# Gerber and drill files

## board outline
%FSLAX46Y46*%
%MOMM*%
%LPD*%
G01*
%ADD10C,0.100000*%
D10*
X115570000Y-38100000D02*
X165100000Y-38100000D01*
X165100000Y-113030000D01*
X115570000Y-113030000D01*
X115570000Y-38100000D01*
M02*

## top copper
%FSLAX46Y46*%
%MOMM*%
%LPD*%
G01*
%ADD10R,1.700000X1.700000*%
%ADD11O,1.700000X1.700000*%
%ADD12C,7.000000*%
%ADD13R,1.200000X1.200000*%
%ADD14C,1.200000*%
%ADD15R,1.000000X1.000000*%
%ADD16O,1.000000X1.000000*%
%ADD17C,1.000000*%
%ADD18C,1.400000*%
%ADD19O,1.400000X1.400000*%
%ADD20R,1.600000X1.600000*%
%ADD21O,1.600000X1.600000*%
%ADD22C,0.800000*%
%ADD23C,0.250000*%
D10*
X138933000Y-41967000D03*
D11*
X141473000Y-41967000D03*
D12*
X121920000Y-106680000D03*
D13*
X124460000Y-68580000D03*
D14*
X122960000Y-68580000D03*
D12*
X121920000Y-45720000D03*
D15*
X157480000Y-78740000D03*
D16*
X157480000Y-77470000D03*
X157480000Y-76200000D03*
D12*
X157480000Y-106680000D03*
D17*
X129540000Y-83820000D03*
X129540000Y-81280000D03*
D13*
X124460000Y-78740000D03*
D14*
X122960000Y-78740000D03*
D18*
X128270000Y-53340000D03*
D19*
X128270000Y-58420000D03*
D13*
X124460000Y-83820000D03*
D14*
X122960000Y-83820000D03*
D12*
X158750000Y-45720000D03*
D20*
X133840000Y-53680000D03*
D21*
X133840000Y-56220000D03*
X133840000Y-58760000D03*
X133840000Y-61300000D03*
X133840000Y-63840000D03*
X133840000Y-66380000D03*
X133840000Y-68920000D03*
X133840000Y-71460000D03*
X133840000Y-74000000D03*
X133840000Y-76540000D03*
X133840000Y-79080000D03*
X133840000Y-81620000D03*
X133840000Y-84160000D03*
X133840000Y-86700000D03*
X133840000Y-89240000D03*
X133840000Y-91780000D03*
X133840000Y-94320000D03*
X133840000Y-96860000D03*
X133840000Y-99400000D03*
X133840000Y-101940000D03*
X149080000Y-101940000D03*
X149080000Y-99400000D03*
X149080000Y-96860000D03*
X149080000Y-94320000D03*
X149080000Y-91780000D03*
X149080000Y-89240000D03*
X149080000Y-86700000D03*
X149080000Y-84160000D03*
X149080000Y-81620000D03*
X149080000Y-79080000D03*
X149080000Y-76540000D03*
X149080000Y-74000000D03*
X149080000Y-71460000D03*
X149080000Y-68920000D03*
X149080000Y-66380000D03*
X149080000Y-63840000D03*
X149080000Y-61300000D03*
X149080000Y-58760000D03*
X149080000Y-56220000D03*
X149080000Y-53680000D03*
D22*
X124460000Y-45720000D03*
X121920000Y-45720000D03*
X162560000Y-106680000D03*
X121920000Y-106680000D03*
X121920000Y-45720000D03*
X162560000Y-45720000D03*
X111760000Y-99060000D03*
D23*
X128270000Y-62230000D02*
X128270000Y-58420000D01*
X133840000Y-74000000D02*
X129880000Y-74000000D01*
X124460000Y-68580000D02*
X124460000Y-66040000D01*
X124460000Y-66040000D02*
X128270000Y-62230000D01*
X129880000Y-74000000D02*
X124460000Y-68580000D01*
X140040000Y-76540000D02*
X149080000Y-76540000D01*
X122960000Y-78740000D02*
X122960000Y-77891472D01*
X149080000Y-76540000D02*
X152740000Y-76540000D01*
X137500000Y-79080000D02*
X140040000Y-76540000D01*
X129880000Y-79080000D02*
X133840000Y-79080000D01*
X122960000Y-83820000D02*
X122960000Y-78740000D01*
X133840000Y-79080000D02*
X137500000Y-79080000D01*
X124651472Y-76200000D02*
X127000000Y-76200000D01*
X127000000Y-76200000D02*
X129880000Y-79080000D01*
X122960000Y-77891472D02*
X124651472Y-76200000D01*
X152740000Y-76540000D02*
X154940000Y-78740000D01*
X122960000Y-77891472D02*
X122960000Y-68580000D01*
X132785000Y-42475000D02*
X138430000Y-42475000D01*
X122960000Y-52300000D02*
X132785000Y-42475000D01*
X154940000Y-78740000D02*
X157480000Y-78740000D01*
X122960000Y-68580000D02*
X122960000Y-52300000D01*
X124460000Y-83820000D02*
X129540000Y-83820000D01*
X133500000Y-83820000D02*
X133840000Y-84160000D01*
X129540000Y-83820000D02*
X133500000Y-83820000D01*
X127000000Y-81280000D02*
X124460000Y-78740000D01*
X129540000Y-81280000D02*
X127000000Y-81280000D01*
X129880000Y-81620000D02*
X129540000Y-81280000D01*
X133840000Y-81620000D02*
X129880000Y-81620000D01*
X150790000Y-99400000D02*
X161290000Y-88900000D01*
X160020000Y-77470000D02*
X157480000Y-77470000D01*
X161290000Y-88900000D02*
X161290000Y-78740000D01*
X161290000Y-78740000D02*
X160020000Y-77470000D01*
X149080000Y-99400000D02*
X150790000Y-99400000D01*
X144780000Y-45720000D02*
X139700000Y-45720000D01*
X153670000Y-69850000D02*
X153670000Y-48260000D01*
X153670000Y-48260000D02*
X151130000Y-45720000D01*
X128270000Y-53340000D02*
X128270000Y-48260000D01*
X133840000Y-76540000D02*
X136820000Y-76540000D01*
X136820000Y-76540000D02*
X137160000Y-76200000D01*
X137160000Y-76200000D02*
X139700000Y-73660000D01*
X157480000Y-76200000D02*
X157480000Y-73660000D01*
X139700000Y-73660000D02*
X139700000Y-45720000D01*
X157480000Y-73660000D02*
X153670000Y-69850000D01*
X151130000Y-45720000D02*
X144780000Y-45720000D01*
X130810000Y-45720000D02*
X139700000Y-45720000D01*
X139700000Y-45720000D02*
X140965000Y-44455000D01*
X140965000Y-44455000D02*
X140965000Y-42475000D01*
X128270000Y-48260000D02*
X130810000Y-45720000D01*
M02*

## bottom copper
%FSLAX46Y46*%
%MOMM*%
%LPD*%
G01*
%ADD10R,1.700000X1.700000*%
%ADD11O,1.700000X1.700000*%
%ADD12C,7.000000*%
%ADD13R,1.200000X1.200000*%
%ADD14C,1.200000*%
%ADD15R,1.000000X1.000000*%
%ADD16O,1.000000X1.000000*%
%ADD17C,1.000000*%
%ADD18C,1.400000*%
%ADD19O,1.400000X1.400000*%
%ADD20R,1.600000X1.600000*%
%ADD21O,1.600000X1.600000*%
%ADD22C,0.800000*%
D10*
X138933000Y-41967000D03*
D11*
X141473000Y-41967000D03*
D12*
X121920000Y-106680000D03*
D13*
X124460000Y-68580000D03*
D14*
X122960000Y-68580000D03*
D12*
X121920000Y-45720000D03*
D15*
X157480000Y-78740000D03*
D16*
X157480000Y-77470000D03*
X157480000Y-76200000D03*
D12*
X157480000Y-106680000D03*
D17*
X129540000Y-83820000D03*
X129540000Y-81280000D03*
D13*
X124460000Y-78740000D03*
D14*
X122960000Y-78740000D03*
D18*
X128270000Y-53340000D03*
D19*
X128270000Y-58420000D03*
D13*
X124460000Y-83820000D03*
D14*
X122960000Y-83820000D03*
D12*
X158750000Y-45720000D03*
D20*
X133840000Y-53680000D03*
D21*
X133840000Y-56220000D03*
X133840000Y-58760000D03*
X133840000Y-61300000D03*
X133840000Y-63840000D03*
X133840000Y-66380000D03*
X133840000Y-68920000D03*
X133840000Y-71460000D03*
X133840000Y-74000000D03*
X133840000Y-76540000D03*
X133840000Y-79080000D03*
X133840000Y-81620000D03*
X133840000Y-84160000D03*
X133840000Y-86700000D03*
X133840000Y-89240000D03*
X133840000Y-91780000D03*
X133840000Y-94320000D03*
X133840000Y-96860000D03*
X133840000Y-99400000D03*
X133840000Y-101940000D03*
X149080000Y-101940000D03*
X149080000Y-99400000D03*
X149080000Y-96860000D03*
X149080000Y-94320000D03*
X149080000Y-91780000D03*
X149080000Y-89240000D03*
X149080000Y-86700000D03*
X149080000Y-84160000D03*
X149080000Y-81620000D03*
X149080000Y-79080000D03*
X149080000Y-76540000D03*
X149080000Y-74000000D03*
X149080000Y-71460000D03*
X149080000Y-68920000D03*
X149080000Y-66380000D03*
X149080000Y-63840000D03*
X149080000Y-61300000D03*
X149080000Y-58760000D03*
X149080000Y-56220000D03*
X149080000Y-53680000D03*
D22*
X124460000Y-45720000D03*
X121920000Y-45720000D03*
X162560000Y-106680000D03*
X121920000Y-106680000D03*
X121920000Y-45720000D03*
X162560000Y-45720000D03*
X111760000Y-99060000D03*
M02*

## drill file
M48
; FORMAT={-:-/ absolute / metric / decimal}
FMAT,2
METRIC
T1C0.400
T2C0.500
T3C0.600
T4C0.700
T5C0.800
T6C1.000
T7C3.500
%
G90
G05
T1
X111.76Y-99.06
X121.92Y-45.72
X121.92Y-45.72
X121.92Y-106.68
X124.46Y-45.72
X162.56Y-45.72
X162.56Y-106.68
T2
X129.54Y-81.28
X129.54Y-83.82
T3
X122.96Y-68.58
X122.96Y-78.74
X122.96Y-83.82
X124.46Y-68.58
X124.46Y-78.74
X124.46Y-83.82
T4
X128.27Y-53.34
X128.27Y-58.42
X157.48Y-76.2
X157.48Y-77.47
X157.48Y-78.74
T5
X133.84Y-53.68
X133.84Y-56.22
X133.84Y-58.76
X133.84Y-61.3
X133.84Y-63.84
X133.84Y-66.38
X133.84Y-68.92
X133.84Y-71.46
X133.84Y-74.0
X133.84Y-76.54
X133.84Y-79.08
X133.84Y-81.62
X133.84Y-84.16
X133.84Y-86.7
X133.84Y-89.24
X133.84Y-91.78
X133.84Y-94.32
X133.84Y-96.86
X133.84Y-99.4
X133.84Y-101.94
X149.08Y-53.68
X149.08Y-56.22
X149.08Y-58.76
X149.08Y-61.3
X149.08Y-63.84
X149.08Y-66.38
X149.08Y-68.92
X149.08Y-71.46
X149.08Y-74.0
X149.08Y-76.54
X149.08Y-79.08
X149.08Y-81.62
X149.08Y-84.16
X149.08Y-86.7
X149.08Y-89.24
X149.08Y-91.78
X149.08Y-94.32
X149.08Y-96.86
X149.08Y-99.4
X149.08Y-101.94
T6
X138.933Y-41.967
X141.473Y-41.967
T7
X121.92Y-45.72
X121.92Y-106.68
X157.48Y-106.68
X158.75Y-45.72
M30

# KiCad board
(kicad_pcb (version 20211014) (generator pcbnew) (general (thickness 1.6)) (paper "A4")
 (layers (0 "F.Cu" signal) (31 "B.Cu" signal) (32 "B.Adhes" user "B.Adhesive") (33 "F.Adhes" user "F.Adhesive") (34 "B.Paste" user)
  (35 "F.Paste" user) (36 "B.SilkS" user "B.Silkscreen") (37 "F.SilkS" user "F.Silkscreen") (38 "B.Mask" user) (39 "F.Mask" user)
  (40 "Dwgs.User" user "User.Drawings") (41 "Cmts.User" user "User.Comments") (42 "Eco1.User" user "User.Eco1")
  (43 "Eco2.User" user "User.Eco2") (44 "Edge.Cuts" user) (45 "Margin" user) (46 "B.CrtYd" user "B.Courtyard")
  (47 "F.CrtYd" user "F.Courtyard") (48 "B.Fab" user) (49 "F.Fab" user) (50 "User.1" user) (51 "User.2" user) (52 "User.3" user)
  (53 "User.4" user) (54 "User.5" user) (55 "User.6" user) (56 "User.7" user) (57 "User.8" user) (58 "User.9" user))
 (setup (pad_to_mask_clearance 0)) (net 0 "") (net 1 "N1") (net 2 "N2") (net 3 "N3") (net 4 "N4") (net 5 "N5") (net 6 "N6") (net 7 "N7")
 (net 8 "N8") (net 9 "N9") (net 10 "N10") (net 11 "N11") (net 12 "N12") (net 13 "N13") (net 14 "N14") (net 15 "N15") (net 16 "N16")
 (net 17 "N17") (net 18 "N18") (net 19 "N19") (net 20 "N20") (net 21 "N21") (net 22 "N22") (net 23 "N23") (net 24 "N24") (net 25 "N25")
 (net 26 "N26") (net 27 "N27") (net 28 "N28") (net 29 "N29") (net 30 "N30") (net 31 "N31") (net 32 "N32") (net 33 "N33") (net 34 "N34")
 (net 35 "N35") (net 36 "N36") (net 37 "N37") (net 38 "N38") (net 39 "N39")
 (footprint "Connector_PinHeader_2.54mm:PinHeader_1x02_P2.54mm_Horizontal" (layer "F.Cu") (at 138.933 41.967 90)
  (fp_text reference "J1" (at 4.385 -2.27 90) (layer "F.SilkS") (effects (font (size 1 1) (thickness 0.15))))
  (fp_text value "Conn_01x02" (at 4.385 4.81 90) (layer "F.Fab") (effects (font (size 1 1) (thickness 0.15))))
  (pad "1" thru_hole rect (at 0 0 90) (size 1.7 1.7) (drill 1) (layers *.Cu *.Mask) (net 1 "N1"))
  (pad "2" thru_hole oval (at 0 2.54 90) (size 1.7 1.7) (drill 1) (layers *.Cu *.Mask) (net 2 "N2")))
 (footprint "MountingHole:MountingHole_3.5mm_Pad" (layer "F.Cu") (at 121.92 106.68)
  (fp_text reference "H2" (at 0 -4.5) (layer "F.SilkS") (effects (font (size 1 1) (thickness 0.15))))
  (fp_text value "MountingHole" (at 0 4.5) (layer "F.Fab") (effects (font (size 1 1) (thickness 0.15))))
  (pad "1" thru_hole circle (at 0 0) (size 7 7) (drill 3.5) (layers *.Cu *.Mask)))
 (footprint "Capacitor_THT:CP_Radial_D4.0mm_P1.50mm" (layer "F.Cu") (at 124.46 68.58 180)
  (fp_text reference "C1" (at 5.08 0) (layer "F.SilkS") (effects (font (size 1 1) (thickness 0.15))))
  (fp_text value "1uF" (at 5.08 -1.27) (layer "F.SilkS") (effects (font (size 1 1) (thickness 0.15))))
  (pad "1" thru_hole rect (at 0 0 180) (size 1.2 1.2) (drill 0.6) (layers *.Cu *.Mask) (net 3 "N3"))
  (pad "2" thru_hole circle (at 1.5 0 180) (size 1.2 1.2) (drill 0.6) (layers *.Cu *.Mask) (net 1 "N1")))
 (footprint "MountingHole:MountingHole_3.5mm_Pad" (layer "F.Cu") (at 121.92 45.72)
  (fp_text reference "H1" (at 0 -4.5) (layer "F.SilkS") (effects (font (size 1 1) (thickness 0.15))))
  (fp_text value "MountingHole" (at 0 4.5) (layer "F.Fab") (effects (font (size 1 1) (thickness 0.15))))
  (pad "1" thru_hole circle (at 0 0) (size 7 7) (drill 3.5) (layers *.Cu *.Mask)))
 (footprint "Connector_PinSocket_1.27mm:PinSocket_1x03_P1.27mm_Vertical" (layer "F.Cu") (at 157.48 78.74 180)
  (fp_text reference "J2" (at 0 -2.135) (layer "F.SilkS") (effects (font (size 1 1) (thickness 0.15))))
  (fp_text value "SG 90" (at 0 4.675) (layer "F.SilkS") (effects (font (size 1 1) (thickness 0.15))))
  (pad "1" thru_hole rect (at 0 0 180) (size 1 1) (drill 0.7) (layers *.Cu *.Mask) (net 1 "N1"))
  (pad "2" thru_hole oval (at 0 1.27 180) (size 1 1) (drill 0.7) (layers *.Cu *.Mask) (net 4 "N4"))
  (pad "3" thru_hole oval (at 0 2.54 180) (size 1 1) (drill 0.7) (layers *.Cu *.Mask) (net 2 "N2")))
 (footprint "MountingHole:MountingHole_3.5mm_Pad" (layer "F.Cu") (at 157.48 106.68)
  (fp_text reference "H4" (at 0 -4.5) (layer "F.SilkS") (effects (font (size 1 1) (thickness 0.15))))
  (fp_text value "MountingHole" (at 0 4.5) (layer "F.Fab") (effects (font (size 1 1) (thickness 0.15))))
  (pad "1" thru_hole circle (at 0 0) (size 7 7) (drill 3.5) (layers *.Cu *.Mask)))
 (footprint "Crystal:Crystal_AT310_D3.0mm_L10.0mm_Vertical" (layer "F.Cu") (at 129.54 83.82 90)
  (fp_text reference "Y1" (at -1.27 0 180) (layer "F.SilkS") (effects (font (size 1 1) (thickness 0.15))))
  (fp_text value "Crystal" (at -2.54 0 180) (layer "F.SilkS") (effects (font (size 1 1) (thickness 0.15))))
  (pad "1" thru_hole circle (at 0 0 90) (size 1 1) (drill 0.5) (layers *.Cu *.Mask) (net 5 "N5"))
  (pad "2" thru_hole circle (at 2.54 0 90) (size 1 1) (drill 0.5) (layers *.Cu *.Mask) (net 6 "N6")))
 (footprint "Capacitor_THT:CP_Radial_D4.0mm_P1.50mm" (layer "F.Cu") (at 124.46 78.74 180)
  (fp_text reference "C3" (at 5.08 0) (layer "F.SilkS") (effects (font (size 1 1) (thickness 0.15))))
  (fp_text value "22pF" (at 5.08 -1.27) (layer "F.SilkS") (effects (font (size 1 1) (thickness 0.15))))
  (pad "1" thru_hole rect (at 0 0 180) (size 1.2 1.2) (drill 0.6) (layers *.Cu *.Mask) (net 6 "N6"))
  (pad "2" thru_hole circle (at 1.5 0 180) (size 1.2 1.2) (drill 0.6) (layers *.Cu *.Mask) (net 1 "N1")))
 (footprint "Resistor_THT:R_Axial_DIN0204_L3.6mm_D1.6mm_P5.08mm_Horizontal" (layer "F.Cu") (at 128.27 53.34 -90)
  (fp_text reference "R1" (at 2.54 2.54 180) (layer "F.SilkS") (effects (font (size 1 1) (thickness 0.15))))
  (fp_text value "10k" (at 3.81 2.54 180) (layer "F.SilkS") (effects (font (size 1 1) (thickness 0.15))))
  (pad "1" thru_hole circle (at 0 0 270) (size 1.4 1.4) (drill 0.7) (layers *.Cu *.Mask) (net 2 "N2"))
  (pad "2" thru_hole oval (at 5.08 0 270) (size 1.4 1.4) (drill 0.7) (layers *.Cu *.Mask) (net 3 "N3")))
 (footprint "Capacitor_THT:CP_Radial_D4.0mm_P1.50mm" (layer "F.Cu") (at 124.46 83.82 180)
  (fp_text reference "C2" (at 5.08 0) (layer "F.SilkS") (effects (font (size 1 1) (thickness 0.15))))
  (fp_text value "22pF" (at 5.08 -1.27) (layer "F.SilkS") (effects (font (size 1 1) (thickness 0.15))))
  (pad "1" thru_hole rect (at 0 0 180) (size 1.2 1.2) (drill 0.6) (layers *.Cu *.Mask) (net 5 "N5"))
  (pad "2" thru_hole circle (at 1.5 0 180) (size 1.2 1.2) (drill 0.6) (layers *.Cu *.Mask) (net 1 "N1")))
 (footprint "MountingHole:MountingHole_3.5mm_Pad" (layer "F.Cu") (at 158.75 45.72)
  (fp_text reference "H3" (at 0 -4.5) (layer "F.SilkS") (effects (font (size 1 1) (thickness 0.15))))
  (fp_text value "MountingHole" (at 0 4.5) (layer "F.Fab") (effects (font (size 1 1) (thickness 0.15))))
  (pad "1" thru_hole circle (at 0 0) (size 7 7) (drill 3.5) (layers *.Cu *.Mask)))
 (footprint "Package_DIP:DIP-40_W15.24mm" (layer "F.Cu") (at 133.84 53.68)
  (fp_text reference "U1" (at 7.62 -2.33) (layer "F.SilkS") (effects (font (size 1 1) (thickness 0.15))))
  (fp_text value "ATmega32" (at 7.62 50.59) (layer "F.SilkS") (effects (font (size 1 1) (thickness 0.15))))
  (pad "1" thru_hole rect (at 0 0) (size 1.6 1.6) (drill 0.8) (layers *.Cu *.Mask) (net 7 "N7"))
  (pad "2" thru_hole oval (at 0 2.54) (size 1.6 1.6) (drill 0.8) (layers *.Cu *.Mask) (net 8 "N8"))
  (pad "3" thru_hole oval (at 0 5.08) (size 1.6 1.6) (drill 0.8) (layers *.Cu *.Mask) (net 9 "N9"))
  (pad "4" thru_hole oval (at 0 7.62) (size 1.6 1.6) (drill 0.8) (layers *.Cu *.Mask) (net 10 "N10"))
  (pad "5" thru_hole oval (at 0 10.16) (size 1.6 1.6) (drill 0.8) (layers *.Cu *.Mask) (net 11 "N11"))
  (pad "6" thru_hole oval (at 0 12.7) (size 1.6 1.6) (drill 0.8) (layers *.Cu *.Mask) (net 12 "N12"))
  (pad "7" thru_hole oval (at 0 15.24) (size 1.6 1.6) (drill 0.8) (layers *.Cu *.Mask) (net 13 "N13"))
  (pad "8" thru_hole oval (at 0 17.78) (size 1.6 1.6) (drill 0.8) (layers *.Cu *.Mask) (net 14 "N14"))
  (pad "9" thru_hole oval (at 0 20.32) (size 1.6 1.6) (drill 0.8) (layers *.Cu *.Mask) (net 3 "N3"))
  (pad "10" thru_hole oval (at 0 22.86) (size 1.6 1.6) (drill 0.8) (layers *.Cu *.Mask) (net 2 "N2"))
  (pad "11" thru_hole oval (at 0 25.4) (size 1.6 1.6) (drill 0.8) (layers *.Cu *.Mask) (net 1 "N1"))
  (pad "12" thru_hole oval (at 0 27.94) (size 1.6 1.6) (drill 0.8) (layers *.Cu *.Mask) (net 6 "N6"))
  (pad "13" thru_hole oval (at 0 30.48) (size 1.6 1.6) (drill 0.8) (layers *.Cu *.Mask) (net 5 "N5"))
  (pad "14" thru_hole oval (at 0 33.02) (size 1.6 1.6) (drill 0.8) (layers *.Cu *.Mask) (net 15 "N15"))
  (pad "15" thru_hole oval (at 0 35.56) (size 1.6 1.6) (drill 0.8) (layers *.Cu *.Mask) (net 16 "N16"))
  (pad "16" thru_hole oval (at 0 38.1) (size 1.6 1.6) (drill 0.8) (layers *.Cu *.Mask) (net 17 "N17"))
  (pad "17" thru_hole oval (at 0 40.64) (size 1.6 1.6) (drill 0.8) (layers *.Cu *.Mask) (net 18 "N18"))
  (pad "18" thru_hole oval (at 0 43.18) (size 1.6 1.6) (drill 0.8) (layers *.Cu *.Mask) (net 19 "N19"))
  (pad "19" thru_hole oval (at 0 45.72) (size 1.6 1.6) (drill 0.8) (layers *.Cu *.Mask) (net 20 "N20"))
  (pad "20" thru_hole oval (at 0 48.26) (size 1.6 1.6) (drill 0.8) (layers *.Cu *.Mask) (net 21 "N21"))
  (pad "21" thru_hole oval (at 15.24 48.26) (size 1.6 1.6) (drill 0.8) (layers *.Cu *.Mask) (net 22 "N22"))
  (pad "22" thru_hole oval (at 15.24 45.72) (size 1.6 1.6) (drill 0.8) (layers *.Cu *.Mask) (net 4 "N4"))
  (pad "23" thru_hole oval (at 15.24 43.18) (size 1.6 1.6) (drill 0.8) (layers *.Cu *.Mask) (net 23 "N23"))
  (pad "24" thru_hole oval (at 15.24 40.64) (size 1.6 1.6) (drill 0.8) (layers *.Cu *.Mask) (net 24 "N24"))
  (pad "25" thru_hole oval (at 15.24 38.1) (size 1.6 1.6) (drill 0.8) (layers *.Cu *.Mask) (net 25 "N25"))
  (pad "26" thru_hole oval (at 15.24 35.56) (size 1.6 1.6) (drill 0.8) (layers *.Cu *.Mask) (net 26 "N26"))
  (pad "27" thru_hole oval (at 15.24 33.02) (size 1.6 1.6) (drill 0.8) (layers *.Cu *.Mask) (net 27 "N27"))
  (pad "28" thru_hole oval (at 15.24 30.48) (size 1.6 1.6) (drill 0.8) (layers *.Cu *.Mask) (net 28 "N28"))
  (pad "29" thru_hole oval (at 15.24 27.94) (size 1.6 1.6) (drill 0.8) (layers *.Cu *.Mask) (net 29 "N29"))
  (pad "30" thru_hole oval (at 15.24 25.4) (size 1.6 1.6) (drill 0.8) (layers *.Cu *.Mask) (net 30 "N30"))
  (pad "31" thru_hole oval (at 15.24 22.86) (size 1.6 1.6) (drill 0.8) (layers *.Cu *.Mask) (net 1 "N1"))
  (pad "32" thru_hole oval (at 15.24 20.32) (size 1.6 1.6) (drill 0.8) (layers *.Cu *.Mask) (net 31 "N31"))
  (pad "33" thru_hole oval (at 15.24 17.78) (size 1.6 1.6) (drill 0.8) (layers *.Cu *.Mask) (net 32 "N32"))
  (pad "34" thru_hole oval (at 15.24 15.24) (size 1.6 1.6) (drill 0.8) (layers *.Cu *.Mask) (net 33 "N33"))
  (pad "35" thru_hole oval (at 15.24 12.7) (size 1.6 1.6) (drill 0.8) (layers *.Cu *.Mask) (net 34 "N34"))
  (pad "36" thru_hole oval (at 15.24 10.16) (size 1.6 1.6) (drill 0.8) (layers *.Cu *.Mask) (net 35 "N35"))
  (pad "37" thru_hole oval (at 15.24 7.62) (size 1.6 1.6) (drill 0.8) (layers *.Cu *.Mask) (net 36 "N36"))
  (pad "38" thru_hole oval (at 15.24 5.08) (size 1.6 1.6) (drill 0.8) (layers *.Cu *.Mask) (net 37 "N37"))
  (pad "39" thru_hole oval (at 15.24 2.54) (size 1.6 1.6) (drill 0.8) (layers *.Cu *.Mask) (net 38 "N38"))
  (pad "40" thru_hole oval (at 15.24 0) (size 1.6 1.6) (drill 0.8) (layers *.Cu *.Mask) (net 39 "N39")))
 (gr_rect (start 115.57 38.1) (end 165.1 113.03) (layer "Edge.Cuts") (width 0.1) (fill none))
 (via (at 124.46 45.72) (size 0.8) (drill 0.4) (layers "F.Cu" "B.Cu") (free) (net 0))
 (via (at 121.92 45.72) (size 0.8) (drill 0.4) (layers "F.Cu" "B.Cu") (free) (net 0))
 (via (at 162.56 106.68) (size 0.8) (drill 0.4) (layers "F.Cu" "B.Cu") (free) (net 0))
 (via (at 121.92 106.68) (size 0.8) (drill 0.4) (layers "F.Cu" "B.Cu") (free) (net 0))
 (via (at 121.92 45.72) (size 0.8) (drill 0.4) (layers "F.Cu" "B.Cu") (free) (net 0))
 (via (at 162.56 45.72) (size 0.8) (drill 0.4) (layers "F.Cu" "B.Cu") (free) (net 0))
 (via (at 111.76 99.06) (size 0.8) (drill 0.4) (layers "F.Cu" "B.Cu") (free) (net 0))
 (segment (start 128.27 62.23) (end 128.27 58.42) (width 0.25) (layer "F.Cu") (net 3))
 (segment (start 133.84 74) (end 129.88 74) (width 0.25) (layer "F.Cu") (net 3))
 (segment (start 124.46 68.58) (end 124.46 66.04) (width 0.25) (layer "F.Cu") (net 3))
 (segment (start 124.46 66.04) (end 128.27 62.23) (width 0.25) (layer "F.Cu") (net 3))
 (segment (start 129.88 74) (end 124.46 68.58) (width 0.25) (layer "F.Cu") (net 3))
 (segment (start 140.04 76.54) (end 149.08 76.54) (width 0.25) (layer "F.Cu") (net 1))
 (segment (start 122.96 78.74) (end 122.96 77.891472) (width 0.25) (layer "F.Cu") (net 1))
 (segment (start 149.08 76.54) (end 152.74 76.54) (width 0.25) (layer "F.Cu") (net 1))
 (segment (start 137.5 79.08) (end 140.04 76.54) (width 0.25) (layer "F.Cu") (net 1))
 (segment (start 129.88 79.08) (end 133.84 79.08) (width 0.25) (layer "F.Cu") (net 1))
 (segment (start 122.96 83.82) (end 122.96 78.74) (width 0.25) (layer "F.Cu") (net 1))
 (segment (start 133.84 79.08) (end 137.5 79.08) (width 0.25) (layer "F.Cu") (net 1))
 (segment (start 124.651472 76.2) (end 127 76.2) (width 0.25) (layer "F.Cu") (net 1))
 (segment (start 127 76.2) (end 129.88 79.08) (width 0.25) (layer "F.Cu") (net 1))
 (segment (start 122.96 77.891472) (end 124.651472 76.2) (width 0.25) (layer "F.Cu") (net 1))
 (segment (start 152.74 76.54) (end 154.94 78.74) (width 0.25) (layer "F.Cu") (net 1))
 (segment (start 122.96 77.891472) (end 122.96 68.58) (width 0.25) (layer "F.Cu") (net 1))
 (segment (start 132.785 42.475) (end 138.43 42.475) (width 0.25) (layer "F.Cu") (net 1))
 (segment (start 122.96 52.3) (end 132.785 42.475) (width 0.25) (layer "F.Cu") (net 1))
 (segment (start 154.94 78.74) (end 157.48 78.74) (width 0.25) (layer "F.Cu") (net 1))
 (segment (start 122.96 68.58) (end 122.96 52.3) (width 0.25) (layer "F.Cu") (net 1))
 (segment (start 124.46 83.82) (end 129.54 83.82) (width 0.25) (layer "F.Cu") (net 5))
 (segment (start 133.5 83.82) (end 133.84 84.16) (width 0.25) (layer "F.Cu") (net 5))
 (segment (start 129.54 83.82) (end 133.5 83.82) (width 0.25) (layer "F.Cu") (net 5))
 (segment (start 127 81.28) (end 124.46 78.74) (width 0.25) (layer "F.Cu") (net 6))
 (segment (start 129.54 81.28) (end 127 81.28) (width 0.25) (layer "F.Cu") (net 6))
 (segment (start 129.88 81.62) (end 129.54 81.28) (width 0.25) (layer "F.Cu") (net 6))
 (segment (start 133.84 81.62) (end 129.88 81.62) (width 0.25) (layer "F.Cu") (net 6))
 (segment (start 150.79 99.4) (end 161.29 88.9) (width 0.25) (layer "F.Cu") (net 4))
 (segment (start 160.02 77.47) (end 157.48 77.47) (width 0.25) (layer "F.Cu") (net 4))
 (segment (start 161.29 88.9) (end 161.29 78.74) (width 0.25) (layer "F.Cu") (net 4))
 (segment (start 161.29 78.74) (end 160.02 77.47) (width 0.25) (layer "F.Cu") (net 4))
 (segment (start 149.08 99.4) (end 150.79 99.4) (width 0.25) (layer "F.Cu") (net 4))
 (segment (start 144.78 45.72) (end 139.7 45.72) (width 0.25) (layer "F.Cu") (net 2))
 (segment (start 153.67 69.85) (end 153.67 48.26) (width 0.25) (layer "F.Cu") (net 2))
 (segment (start 153.67 48.26) (end 151.13 45.72) (width 0.25) (layer "F.Cu") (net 2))
 (segment (start 128.27 53.34) (end 128.27 48.26) (width 0.25) (layer "F.Cu") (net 2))
 (segment (start 133.84 76.54) (end 136.82 76.54) (width 0.25) (layer "F.Cu") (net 2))
 (segment (start 136.82 76.54) (end 137.16 76.2) (width 0.25) (layer "F.Cu") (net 2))
 (segment (start 137.16 76.2) (end 139.7 73.66) (width 0.25) (layer "F.Cu") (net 2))
 (segment (start 157.48 76.2) (end 157.48 73.66) (width 0.25) (layer "F.Cu") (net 2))
 (segment (start 139.7 73.66) (end 139.7 45.72) (width 0.25) (layer "F.Cu") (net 2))
 (segment (start 157.48 73.66) (end 153.67 69.85) (width 0.25) (layer "F.Cu") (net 2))
 (segment (start 151.13 45.72) (end 144.78 45.72) (width 0.25) (layer "F.Cu") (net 2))
 (segment (start 130.81 45.72) (end 139.7 45.72) (width 0.25) (layer "F.Cu") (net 2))
 (segment (start 139.7 45.72) (end 140.965 44.455) (width 0.25) (layer "F.Cu") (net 2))
 (segment (start 140.965 44.455) (end 140.965 42.475) (width 0.25) (layer "F.Cu") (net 2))
 (segment (start 128.27 48.26) (end 130.81 45.72) (width 0.25) (layer "F.Cu") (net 2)))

